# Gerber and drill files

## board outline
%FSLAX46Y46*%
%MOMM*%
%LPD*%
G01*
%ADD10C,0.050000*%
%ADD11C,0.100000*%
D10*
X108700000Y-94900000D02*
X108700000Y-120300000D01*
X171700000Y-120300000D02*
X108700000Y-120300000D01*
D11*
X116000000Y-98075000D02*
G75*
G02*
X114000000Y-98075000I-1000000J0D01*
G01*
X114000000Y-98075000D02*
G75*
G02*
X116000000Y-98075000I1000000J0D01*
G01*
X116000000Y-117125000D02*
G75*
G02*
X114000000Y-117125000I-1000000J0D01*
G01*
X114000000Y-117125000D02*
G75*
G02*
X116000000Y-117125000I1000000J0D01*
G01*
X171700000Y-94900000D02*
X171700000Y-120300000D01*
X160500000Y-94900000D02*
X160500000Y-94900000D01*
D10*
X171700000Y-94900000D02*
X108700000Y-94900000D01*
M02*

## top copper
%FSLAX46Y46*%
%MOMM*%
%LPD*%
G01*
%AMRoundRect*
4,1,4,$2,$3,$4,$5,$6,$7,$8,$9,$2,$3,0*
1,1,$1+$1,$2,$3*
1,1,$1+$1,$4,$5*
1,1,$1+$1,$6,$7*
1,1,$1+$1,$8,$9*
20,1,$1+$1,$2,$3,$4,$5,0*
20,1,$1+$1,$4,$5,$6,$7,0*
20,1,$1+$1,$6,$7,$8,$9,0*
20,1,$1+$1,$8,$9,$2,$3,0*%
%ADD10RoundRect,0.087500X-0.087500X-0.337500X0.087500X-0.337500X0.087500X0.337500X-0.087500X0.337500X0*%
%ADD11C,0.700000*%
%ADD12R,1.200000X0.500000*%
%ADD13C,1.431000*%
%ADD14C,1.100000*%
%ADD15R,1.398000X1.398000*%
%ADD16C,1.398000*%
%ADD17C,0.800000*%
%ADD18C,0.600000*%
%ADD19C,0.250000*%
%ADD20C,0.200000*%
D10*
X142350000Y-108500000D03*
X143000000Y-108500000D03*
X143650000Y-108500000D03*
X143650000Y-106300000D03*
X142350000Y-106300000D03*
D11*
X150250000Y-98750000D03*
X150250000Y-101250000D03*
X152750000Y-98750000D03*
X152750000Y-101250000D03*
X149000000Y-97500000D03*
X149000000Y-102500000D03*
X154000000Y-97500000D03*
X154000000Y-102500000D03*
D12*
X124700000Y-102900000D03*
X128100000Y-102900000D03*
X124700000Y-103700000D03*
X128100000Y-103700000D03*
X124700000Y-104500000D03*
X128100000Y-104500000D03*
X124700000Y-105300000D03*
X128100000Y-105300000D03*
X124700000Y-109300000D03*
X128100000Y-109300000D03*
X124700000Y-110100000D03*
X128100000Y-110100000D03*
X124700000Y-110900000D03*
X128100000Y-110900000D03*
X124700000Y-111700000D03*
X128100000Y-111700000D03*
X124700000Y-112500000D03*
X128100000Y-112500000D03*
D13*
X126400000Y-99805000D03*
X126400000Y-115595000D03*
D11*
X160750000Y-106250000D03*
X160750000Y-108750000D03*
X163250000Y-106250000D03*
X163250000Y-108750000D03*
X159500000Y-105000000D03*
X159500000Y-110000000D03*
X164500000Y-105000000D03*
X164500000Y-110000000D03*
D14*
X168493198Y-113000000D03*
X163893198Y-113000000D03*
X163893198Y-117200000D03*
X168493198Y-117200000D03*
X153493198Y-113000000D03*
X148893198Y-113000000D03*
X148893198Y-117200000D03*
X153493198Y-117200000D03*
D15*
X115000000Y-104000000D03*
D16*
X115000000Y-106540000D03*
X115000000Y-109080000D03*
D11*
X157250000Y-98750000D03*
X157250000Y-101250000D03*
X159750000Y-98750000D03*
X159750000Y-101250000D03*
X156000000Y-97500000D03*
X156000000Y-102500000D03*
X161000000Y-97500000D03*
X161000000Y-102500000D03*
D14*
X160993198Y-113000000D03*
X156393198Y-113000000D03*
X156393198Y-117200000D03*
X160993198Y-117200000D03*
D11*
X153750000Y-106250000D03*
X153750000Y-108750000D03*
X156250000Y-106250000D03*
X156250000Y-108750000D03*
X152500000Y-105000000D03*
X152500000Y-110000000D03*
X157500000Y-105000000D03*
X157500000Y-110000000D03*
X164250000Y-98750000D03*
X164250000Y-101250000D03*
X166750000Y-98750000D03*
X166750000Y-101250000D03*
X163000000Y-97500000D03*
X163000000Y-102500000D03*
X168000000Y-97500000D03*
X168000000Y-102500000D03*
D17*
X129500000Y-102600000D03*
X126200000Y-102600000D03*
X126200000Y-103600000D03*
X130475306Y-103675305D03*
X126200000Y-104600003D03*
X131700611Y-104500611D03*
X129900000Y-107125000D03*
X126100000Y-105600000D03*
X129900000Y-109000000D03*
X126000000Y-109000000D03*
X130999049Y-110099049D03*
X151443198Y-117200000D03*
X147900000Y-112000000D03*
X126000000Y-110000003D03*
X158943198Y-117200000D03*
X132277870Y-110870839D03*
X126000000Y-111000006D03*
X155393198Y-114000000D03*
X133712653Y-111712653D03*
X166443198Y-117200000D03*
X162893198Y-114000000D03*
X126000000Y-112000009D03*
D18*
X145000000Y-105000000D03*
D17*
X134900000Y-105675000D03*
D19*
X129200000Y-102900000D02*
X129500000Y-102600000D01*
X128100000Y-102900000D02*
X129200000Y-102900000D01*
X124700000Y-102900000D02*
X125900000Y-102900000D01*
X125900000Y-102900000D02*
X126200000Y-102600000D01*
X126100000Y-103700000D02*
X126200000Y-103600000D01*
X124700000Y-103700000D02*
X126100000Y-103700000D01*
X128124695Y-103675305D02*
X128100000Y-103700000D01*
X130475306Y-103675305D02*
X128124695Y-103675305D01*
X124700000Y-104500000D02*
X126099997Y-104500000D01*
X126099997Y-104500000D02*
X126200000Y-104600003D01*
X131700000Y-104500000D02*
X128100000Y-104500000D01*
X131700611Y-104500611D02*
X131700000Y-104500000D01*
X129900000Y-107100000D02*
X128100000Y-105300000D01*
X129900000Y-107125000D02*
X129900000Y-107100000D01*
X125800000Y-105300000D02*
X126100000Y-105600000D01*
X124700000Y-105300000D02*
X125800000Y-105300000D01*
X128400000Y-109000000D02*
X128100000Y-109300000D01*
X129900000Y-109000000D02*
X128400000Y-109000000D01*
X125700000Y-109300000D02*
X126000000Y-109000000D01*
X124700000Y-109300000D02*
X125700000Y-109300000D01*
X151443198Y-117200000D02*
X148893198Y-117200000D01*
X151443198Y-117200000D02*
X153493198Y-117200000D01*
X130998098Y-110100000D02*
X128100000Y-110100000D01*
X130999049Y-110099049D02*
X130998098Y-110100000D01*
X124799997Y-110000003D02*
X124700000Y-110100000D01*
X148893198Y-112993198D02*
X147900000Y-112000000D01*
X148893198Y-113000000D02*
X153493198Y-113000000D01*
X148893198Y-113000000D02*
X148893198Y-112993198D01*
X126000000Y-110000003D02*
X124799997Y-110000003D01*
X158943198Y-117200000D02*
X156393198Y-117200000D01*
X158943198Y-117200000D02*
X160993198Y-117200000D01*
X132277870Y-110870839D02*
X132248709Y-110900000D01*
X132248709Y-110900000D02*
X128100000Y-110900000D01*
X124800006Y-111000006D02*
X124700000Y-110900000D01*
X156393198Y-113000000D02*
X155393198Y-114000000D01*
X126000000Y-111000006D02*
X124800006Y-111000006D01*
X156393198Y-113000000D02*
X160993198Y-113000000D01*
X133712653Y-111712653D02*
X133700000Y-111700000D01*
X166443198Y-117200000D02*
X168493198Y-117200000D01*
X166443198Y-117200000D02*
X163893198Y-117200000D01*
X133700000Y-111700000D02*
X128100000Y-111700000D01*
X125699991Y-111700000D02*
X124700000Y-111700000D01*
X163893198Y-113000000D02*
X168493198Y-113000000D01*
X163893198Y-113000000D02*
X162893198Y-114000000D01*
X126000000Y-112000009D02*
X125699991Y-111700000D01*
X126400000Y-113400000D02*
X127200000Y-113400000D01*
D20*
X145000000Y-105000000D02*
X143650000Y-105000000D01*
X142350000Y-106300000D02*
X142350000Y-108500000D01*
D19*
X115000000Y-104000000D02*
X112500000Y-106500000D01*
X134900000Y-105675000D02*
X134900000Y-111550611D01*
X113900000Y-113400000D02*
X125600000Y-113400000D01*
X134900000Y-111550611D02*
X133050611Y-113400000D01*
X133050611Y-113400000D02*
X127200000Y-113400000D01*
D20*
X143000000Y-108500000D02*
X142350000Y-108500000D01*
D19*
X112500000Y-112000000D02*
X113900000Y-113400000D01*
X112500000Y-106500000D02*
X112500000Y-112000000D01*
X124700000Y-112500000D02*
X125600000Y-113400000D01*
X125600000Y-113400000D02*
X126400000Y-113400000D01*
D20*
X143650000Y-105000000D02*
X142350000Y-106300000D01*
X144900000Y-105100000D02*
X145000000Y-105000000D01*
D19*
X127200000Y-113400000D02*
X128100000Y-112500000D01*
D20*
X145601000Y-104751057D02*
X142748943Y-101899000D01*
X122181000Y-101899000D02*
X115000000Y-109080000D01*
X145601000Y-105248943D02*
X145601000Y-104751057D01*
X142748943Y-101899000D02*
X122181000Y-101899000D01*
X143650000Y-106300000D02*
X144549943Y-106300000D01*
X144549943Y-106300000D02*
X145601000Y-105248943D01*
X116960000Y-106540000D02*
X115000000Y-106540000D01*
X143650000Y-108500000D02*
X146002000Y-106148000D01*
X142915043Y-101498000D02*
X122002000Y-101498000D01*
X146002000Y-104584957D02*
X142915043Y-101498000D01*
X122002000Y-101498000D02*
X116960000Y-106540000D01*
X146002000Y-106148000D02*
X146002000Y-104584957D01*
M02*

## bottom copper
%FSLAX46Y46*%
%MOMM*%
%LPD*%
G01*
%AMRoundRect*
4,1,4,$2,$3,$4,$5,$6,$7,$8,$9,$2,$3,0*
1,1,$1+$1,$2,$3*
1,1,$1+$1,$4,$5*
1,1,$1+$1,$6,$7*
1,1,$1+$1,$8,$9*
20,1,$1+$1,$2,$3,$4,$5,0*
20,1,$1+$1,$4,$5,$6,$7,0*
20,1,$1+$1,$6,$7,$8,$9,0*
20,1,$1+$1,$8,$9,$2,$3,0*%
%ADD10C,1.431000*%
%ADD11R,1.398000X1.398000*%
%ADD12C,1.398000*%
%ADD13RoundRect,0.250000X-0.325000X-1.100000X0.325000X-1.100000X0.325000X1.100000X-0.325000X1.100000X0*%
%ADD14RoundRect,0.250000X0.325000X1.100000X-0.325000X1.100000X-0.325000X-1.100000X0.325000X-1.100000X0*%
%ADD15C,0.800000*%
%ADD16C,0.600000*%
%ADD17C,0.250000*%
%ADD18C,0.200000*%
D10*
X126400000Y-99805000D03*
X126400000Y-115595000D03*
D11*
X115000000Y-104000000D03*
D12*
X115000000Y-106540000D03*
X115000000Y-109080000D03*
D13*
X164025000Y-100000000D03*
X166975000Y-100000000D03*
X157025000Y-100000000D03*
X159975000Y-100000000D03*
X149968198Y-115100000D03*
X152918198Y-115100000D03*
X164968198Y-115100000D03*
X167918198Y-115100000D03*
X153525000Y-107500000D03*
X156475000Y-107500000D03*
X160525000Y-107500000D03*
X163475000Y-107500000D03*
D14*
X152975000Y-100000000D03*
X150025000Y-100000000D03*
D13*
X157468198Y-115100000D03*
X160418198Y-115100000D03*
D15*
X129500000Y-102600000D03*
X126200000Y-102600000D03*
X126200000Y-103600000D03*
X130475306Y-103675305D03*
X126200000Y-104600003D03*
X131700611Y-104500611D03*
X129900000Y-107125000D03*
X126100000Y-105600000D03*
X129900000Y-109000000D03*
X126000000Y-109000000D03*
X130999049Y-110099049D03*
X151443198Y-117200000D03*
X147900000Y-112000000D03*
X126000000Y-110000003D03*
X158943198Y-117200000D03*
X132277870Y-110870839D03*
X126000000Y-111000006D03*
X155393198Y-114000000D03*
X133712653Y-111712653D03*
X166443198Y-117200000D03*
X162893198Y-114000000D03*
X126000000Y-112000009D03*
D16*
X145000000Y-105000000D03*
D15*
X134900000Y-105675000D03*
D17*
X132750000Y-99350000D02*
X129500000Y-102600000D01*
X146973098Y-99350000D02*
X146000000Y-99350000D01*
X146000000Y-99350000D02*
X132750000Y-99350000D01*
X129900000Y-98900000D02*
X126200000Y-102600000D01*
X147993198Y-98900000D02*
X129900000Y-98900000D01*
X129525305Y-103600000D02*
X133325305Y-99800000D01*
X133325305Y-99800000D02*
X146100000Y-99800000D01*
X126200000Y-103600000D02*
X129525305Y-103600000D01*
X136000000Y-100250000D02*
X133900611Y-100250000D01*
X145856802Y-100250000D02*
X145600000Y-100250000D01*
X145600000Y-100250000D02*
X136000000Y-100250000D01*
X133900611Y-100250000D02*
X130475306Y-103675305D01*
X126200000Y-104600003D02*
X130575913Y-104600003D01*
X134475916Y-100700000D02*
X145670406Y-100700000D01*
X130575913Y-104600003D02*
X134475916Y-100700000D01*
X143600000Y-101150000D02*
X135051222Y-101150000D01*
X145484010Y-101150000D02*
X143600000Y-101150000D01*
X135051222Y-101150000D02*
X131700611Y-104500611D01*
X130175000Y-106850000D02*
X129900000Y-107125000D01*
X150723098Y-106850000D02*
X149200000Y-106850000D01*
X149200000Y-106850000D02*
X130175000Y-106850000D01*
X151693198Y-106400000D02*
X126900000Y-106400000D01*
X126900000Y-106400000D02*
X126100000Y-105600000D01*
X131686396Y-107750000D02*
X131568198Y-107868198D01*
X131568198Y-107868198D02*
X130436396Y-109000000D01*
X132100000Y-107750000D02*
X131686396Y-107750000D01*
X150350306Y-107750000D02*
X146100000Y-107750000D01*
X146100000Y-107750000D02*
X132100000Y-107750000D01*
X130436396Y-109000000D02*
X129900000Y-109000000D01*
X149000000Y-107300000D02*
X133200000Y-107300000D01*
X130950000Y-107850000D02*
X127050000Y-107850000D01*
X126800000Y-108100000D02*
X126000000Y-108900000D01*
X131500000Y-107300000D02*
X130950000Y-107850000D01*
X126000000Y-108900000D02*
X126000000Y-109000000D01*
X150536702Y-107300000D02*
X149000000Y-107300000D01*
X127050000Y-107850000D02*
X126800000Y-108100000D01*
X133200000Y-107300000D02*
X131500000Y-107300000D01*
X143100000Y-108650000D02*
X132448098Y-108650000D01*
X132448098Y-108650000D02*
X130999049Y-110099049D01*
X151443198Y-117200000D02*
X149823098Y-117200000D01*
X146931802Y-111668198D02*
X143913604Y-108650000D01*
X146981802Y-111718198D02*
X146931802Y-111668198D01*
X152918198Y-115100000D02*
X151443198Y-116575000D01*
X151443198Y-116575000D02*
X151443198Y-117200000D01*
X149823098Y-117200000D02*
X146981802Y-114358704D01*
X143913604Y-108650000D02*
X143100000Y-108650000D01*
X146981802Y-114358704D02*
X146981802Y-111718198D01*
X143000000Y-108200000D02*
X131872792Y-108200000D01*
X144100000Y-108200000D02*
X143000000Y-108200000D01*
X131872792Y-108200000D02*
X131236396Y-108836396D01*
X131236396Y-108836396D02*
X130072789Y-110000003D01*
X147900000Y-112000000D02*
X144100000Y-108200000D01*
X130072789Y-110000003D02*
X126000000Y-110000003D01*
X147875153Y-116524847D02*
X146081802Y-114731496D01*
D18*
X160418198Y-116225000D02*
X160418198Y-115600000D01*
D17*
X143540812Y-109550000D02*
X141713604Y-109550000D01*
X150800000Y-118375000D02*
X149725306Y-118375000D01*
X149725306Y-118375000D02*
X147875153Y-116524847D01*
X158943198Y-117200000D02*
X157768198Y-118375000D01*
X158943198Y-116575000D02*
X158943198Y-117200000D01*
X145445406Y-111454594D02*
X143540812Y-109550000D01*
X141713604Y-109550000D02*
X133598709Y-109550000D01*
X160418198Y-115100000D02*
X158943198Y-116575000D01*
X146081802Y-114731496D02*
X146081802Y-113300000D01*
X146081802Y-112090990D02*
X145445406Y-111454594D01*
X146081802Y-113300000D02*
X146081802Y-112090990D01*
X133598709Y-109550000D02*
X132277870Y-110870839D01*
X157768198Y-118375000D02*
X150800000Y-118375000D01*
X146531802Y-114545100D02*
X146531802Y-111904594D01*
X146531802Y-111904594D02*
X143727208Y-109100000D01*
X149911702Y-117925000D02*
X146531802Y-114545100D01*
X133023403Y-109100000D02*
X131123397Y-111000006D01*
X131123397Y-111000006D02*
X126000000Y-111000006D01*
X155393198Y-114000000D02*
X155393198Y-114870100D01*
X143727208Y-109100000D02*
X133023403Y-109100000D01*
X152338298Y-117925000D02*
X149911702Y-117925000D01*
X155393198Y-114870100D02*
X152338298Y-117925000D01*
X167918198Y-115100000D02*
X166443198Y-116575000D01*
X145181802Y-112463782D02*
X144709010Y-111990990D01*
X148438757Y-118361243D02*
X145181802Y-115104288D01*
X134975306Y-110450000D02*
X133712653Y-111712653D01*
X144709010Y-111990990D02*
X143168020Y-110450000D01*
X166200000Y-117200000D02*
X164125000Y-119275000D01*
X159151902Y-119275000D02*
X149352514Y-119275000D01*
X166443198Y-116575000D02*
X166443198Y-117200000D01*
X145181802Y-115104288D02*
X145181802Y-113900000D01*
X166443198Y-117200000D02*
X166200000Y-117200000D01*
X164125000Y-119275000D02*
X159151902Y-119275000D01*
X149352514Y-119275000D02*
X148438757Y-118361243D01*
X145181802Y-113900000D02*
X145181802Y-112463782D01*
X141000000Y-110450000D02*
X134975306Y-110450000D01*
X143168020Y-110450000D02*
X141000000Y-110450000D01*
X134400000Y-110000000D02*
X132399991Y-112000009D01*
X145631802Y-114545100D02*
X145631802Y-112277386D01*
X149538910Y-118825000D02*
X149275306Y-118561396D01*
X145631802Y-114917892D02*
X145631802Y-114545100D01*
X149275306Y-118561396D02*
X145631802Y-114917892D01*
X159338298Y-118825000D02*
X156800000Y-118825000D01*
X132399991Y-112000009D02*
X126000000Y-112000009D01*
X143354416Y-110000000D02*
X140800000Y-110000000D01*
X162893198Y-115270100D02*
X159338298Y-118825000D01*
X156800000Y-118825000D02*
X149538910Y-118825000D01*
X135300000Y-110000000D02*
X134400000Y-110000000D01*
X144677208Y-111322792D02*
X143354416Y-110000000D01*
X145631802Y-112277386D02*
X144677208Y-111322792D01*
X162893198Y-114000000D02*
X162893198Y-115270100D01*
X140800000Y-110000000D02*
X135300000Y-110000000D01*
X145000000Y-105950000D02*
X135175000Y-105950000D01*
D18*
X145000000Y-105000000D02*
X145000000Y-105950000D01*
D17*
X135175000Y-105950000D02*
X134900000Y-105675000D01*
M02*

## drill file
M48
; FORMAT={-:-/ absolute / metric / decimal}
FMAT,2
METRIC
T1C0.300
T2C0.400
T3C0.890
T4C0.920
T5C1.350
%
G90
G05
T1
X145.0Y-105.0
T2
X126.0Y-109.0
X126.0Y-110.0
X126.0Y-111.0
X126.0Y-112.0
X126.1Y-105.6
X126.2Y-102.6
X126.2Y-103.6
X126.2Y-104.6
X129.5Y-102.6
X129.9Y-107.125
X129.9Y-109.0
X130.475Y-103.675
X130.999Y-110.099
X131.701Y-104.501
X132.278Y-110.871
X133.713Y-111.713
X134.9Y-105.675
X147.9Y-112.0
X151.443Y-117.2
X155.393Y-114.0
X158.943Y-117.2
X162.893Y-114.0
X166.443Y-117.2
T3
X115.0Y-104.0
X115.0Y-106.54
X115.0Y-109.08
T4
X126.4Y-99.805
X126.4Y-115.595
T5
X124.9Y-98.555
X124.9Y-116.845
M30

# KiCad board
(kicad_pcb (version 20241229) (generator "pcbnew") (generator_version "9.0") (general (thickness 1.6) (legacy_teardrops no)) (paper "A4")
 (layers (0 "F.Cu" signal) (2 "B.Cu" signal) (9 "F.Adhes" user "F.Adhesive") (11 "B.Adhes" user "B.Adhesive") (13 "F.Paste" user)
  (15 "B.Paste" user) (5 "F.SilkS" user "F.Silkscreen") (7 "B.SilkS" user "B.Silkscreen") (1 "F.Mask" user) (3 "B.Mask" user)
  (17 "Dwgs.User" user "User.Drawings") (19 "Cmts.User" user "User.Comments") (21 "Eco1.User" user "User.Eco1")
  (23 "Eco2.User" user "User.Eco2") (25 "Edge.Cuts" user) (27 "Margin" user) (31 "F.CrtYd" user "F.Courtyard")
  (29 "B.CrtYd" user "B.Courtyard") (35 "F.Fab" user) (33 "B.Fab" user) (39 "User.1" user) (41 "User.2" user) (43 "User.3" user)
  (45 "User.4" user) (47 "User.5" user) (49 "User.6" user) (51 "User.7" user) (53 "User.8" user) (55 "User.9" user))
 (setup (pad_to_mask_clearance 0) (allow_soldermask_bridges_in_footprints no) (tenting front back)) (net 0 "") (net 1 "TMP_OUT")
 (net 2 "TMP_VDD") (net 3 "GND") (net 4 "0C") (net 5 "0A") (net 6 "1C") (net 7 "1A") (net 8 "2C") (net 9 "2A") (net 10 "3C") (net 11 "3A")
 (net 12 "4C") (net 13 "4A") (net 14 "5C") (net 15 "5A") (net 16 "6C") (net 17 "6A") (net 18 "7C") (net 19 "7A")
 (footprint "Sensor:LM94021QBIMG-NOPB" (layer "F.Cu") (at 143 107.4)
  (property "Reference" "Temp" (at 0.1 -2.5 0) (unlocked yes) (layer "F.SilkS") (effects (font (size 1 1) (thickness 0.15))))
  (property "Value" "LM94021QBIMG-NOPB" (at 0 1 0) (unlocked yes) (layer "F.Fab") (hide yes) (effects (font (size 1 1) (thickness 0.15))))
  (pad "1" smd roundrect (at -0.65 1.1) (size 0.35 0.85) (layers "F.Cu" "F.Mask" "F.Paste") (roundrect_rratio 0.25))
  (pad "2" smd roundrect (at 0 1.1) (size 0.35 0.85) (layers "F.Cu" "F.Mask" "F.Paste") (roundrect_rratio 0.25))
  (pad "3" smd roundrect (at 0.65 1.1) (size 0.35 0.85) (layers "F.Cu" "F.Mask" "F.Paste") (roundrect_rratio 0.25) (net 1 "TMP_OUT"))
  (pad "4" smd roundrect (at 0.65 -1.1) (size 0.35 0.85) (layers "F.Cu" "F.Mask" "F.Paste") (roundrect_rratio 0.25) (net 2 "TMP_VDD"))
  (pad "5" smd roundrect (at -0.65 -1.1) (size 0.35 0.85) (layers "F.Cu" "F.Mask" "F.Paste") (roundrect_rratio 0.25) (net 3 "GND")))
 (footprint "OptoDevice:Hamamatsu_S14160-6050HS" (layer "F.Cu") (at 151.5 100)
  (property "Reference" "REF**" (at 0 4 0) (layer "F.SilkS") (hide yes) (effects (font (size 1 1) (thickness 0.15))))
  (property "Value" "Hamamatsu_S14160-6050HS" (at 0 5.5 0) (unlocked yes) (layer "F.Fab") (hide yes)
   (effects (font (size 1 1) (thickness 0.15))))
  (pad "A" smd circle (at -1.25 -1.25) (size 0.7 0.7) (layers "F.Cu" "F.Mask" "F.Paste"))
  (pad "A" smd circle (at -1.25 1.25) (size 0.7 0.7) (layers "F.Cu" "F.Mask" "F.Paste"))
  (pad "A" smd circle (at 1.25 -1.25) (size 0.7 0.7) (layers "F.Cu" "F.Mask" "F.Paste"))
  (pad "A" smd circle (at 1.25 1.25) (size 0.7 0.7) (layers "F.Cu" "F.Mask" "F.Paste"))
  (pad "K" smd circle (at -2.5 -2.5) (size 0.7 0.7) (layers "F.Cu" "F.Mask" "F.Paste"))
  (pad "K" smd circle (at -2.5 2.5) (size 0.7 0.7) (layers "F.Cu" "F.Mask" "F.Paste"))
  (pad "K" smd circle (at 2.5 -2.5) (size 0.7 0.7) (layers "F.Cu" "F.Mask" "F.Paste"))
  (pad "K" smd circle (at 2.5 2.5) (size 0.7 0.7) (layers "F.Cu" "F.Mask" "F.Paste")))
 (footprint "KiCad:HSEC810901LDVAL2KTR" (layer "F.Cu") (at 126.4 107.7 -90)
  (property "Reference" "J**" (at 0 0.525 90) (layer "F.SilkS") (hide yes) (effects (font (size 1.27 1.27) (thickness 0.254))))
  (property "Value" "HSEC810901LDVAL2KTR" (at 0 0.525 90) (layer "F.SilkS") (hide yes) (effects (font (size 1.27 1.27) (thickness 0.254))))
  (pad "" np_thru_hole circle (at -9.145 1.5 270) (size 1.35 1.35) (drill 1.35) (layers "*.Cu" "*.Mask"))
  (pad "" np_thru_hole circle (at 9.145 1.5 270) (size 1.35 1.35) (drill 1.35) (layers "*.Cu" "*.Mask"))
  (pad "1" smd rect (at -4.8 1.7 270) (size 0.5 1.2) (layers "F.Cu" "F.Mask" "F.Paste") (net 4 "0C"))
  (pad "2" smd rect (at -4.8 -1.7 270) (size 0.5 1.2) (layers "F.Cu" "F.Mask" "F.Paste") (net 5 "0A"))
  (pad "3" smd rect (at -4 1.7 270) (size 0.5 1.2) (layers "F.Cu" "F.Mask" "F.Paste") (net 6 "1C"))
  (pad "4" smd rect (at -4 -1.7 270) (size 0.5 1.2) (layers "F.Cu" "F.Mask" "F.Paste") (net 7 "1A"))
  (pad "5" smd rect (at -3.2 1.7 270) (size 0.5 1.2) (layers "F.Cu" "F.Mask" "F.Paste") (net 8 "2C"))
  (pad "6" smd rect (at -3.2 -1.7 270) (size 0.5 1.2) (layers "F.Cu" "F.Mask" "F.Paste") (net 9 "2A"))
  (pad "7" smd rect (at -2.4 1.7 270) (size 0.5 1.2) (layers "F.Cu" "F.Mask" "F.Paste") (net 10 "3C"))
  (pad "8" smd rect (at -2.4 -1.7 270) (size 0.5 1.2) (layers "F.Cu" "F.Mask" "F.Paste") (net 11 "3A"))
  (pad "9" smd rect (at 1.6 1.7 270) (size 0.5 1.2) (layers "F.Cu" "F.Mask" "F.Paste") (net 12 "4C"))
  (pad "10" smd rect (at 1.6 -1.7 270) (size 0.5 1.2) (layers "F.Cu" "F.Mask" "F.Paste") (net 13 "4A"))
  (pad "11" smd rect (at 2.4 1.7 270) (size 0.5 1.2) (layers "F.Cu" "F.Mask" "F.Paste") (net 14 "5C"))
  (pad "12" smd rect (at 2.4 -1.7 270) (size 0.5 1.2) (layers "F.Cu" "F.Mask" "F.Paste") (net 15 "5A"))
  (pad "13" smd rect (at 3.2 1.7 270) (size 0.5 1.2) (layers "F.Cu" "F.Mask" "F.Paste") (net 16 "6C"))
  (pad "14" smd rect (at 3.2 -1.7 270) (size 0.5 1.2) (layers "F.Cu" "F.Mask" "F.Paste") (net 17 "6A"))
  (pad "15" smd rect (at 4 1.7 270) (size 0.5 1.2) (layers "F.Cu" "F.Mask" "F.Paste") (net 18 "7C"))
  (pad "16" smd rect (at 4 -1.7 270) (size 0.5 1.2) (layers "F.Cu" "F.Mask" "F.Paste") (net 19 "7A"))
  (pad "17" smd rect (at 4.8 1.7 270) (size 0.5 1.2) (layers "F.Cu" "F.Mask" "F.Paste") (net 3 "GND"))
  (pad "18" smd rect (at 4.8 -1.7 270) (size 0.5 1.2) (layers "F.Cu" "F.Mask" "F.Paste") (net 3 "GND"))
  (pad "MH1" thru_hole circle (at -7.895 0 270) (size 1.431 1.431) (drill 0.92) (layers "*.Cu" "*.Mask") (remove_unused_layers no))
  (pad "MH2" thru_hole circle (at 7.895 0 270) (size 1.431 1.431) (drill 0.92) (layers "*.Cu" "*.Mask") (remove_unused_layers no)))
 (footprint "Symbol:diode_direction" (layer "F.Cu") (at 150.243198 107.6 90)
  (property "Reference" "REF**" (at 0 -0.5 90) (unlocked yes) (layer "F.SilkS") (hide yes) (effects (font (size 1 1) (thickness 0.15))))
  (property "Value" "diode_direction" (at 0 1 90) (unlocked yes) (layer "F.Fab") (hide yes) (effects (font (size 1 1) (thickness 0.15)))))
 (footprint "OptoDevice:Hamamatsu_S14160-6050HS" (layer "F.Cu") (at 162 107.5)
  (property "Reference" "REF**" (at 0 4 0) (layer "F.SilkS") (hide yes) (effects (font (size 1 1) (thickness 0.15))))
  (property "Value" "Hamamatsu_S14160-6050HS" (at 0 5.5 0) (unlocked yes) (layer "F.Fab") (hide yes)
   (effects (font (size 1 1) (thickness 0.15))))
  (pad "A" smd circle (at -1.25 -1.25) (size 0.7 0.7) (layers "F.Cu" "F.Mask" "F.Paste"))
  (pad "A" smd circle (at -1.25 1.25) (size 0.7 0.7) (layers "F.Cu" "F.Mask" "F.Paste"))
  (pad "A" smd circle (at 1.25 -1.25) (size 0.7 0.7) (layers "F.Cu" "F.Mask" "F.Paste"))
  (pad "A" smd circle (at 1.25 1.25) (size 0.7 0.7) (layers "F.Cu" "F.Mask" "F.Paste"))
  (pad "K" smd circle (at -2.5 -2.5) (size 0.7 0.7) (layers "F.Cu" "F.Mask" "F.Paste"))
  (pad "K" smd circle (at -2.5 2.5) (size 0.7 0.7) (layers "F.Cu" "F.Mask" "F.Paste"))
  (pad "K" smd circle (at 2.5 -2.5) (size 0.7 0.7) (layers "F.Cu" "F.Mask" "F.Paste"))
  (pad "K" smd circle (at 2.5 2.5) (size 0.7 0.7) (layers "F.Cu" "F.Mask" "F.Paste")))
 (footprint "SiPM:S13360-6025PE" (layer "F.Cu") (at 166.443198 115.1)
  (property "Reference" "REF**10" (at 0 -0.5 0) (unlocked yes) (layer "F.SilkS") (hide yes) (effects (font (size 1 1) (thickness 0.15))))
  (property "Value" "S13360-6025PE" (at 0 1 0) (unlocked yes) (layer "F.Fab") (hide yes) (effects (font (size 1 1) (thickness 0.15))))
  (pad "1" smd circle (at 2.05 -2.1) (size 1.1 1.1) (layers "F.Cu" "F.Mask" "F.Paste") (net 18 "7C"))
  (pad "2" smd circle (at -2.55 -2.1) (size 1.1 1.1) (layers "F.Cu" "F.Mask" "F.Paste") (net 18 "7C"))
  (pad "3" smd circle (at -2.55 2.1) (size 1.1 1.1) (layers "F.Cu" "F.Mask" "F.Paste") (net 19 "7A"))
  (pad "4" smd circle (at 2.05 2.1) (size 1.1 1.1) (layers "F.Cu" "F.Mask" "F.Paste") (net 19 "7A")))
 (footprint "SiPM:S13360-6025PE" (layer "F.Cu") (at 151.443198 115.1)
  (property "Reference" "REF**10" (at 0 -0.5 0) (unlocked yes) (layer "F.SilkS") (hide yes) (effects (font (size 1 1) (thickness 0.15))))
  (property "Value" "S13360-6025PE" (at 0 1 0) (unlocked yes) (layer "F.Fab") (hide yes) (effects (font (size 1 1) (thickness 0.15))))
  (pad "1" smd circle (at 2.05 -2.1) (size 1.1 1.1) (layers "F.Cu" "F.Mask" "F.Paste") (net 14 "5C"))
  (pad "2" smd circle (at -2.55 -2.1) (size 1.1 1.1) (layers "F.Cu" "F.Mask" "F.Paste") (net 14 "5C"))
  (pad "3" smd circle (at -2.55 2.1) (size 1.1 1.1) (layers "F.Cu" "F.Mask" "F.Paste") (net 15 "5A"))
  (pad "4" smd circle (at 2.05 2.1) (size 1.1 1.1) (layers "F.Cu" "F.Mask" "F.Paste") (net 15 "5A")))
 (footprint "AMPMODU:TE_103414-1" (layer "F.Cu") (at 115 106.54 -90)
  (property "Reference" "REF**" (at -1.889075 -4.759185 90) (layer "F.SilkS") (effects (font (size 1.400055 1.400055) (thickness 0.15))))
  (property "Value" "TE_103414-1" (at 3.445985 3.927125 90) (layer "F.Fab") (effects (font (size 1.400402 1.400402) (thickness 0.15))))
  (pad "1" thru_hole rect (at -2.54 0 270) (size 1.398 1.398) (drill 0.89) (layers "*.Cu" "*.Mask") (remove_unused_layers no) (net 3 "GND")
   (solder_mask_margin 0.102))
  (pad "2" thru_hole circle (at 0 0 270) (size 1.398 1.398) (drill 0.89) (layers "*.Cu" "*.Mask") (remove_unused_layers no)
   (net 1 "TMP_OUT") (solder_mask_margin 0.102))
  (pad "3" thru_hole circle (at 2.54 0 270) (size 1.398 1.398) (drill 0.89) (layers "*.Cu" "*.Mask") (remove_unused_layers no)
   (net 2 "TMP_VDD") (solder_mask_margin 0.102)))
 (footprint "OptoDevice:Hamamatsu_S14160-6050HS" (layer "F.Cu") (at 158.5 100)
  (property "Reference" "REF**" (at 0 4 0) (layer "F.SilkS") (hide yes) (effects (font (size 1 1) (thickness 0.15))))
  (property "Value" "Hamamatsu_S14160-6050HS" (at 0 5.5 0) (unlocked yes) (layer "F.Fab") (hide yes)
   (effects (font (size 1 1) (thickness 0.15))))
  (pad "A" smd circle (at -1.25 -1.25) (size 0.7 0.7) (layers "F.Cu" "F.Mask" "F.Paste"))
  (pad "A" smd circle (at -1.25 1.25) (size 0.7 0.7) (layers "F.Cu" "F.Mask" "F.Paste"))
  (pad "A" smd circle (at 1.25 -1.25) (size 0.7 0.7) (layers "F.Cu" "F.Mask" "F.Paste"))
  (pad "A" smd circle (at 1.25 1.25) (size 0.7 0.7) (layers "F.Cu" "F.Mask" "F.Paste"))
  (pad "K" smd circle (at -2.5 -2.5) (size 0.7 0.7) (layers "F.Cu" "F.Mask" "F.Paste"))
  (pad "K" smd circle (at -2.5 2.5) (size 0.7 0.7) (layers "F.Cu" "F.Mask" "F.Paste"))
  (pad "K" smd circle (at 2.5 -2.5) (size 0.7 0.7) (layers "F.Cu" "F.Mask" "F.Paste"))
  (pad "K" smd circle (at 2.5 2.5) (size 0.7 0.7) (layers "F.Cu" "F.Mask" "F.Paste")))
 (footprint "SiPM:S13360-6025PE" (layer "F.Cu") (at 158.943198 115.1)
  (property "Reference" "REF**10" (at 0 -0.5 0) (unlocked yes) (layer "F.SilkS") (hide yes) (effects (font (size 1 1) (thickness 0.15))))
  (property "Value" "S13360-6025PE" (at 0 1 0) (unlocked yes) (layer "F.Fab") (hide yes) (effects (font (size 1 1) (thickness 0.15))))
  (pad "1" smd circle (at 2.05 -2.1) (size 1.1 1.1) (layers "F.Cu" "F.Mask" "F.Paste") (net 16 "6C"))
  (pad "2" smd circle (at -2.55 -2.1) (size 1.1 1.1) (layers "F.Cu" "F.Mask" "F.Paste") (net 16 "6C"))
  (pad "3" smd circle (at -2.55 2.1) (size 1.1 1.1) (layers "F.Cu" "F.Mask" "F.Paste") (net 17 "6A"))
  (pad "4" smd circle (at 2.05 2.1) (size 1.1 1.1) (layers "F.Cu" "F.Mask" "F.Paste") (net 17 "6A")))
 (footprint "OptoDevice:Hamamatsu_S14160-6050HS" (layer "F.Cu") (at 155 107.5)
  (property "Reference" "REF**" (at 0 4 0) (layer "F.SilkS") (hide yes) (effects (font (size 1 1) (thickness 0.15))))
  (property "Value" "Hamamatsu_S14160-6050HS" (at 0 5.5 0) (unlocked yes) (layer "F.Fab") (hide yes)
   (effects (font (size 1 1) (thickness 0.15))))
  (pad "A" smd circle (at -1.25 -1.25) (size 0.7 0.7) (layers "F.Cu" "F.Mask" "F.Paste"))
  (pad "A" smd circle (at -1.25 1.25) (size 0.7 0.7) (layers "F.Cu" "F.Mask" "F.Paste"))
  (pad "A" smd circle (at 1.25 -1.25) (size 0.7 0.7) (layers "F.Cu" "F.Mask" "F.Paste"))
  (pad "A" smd circle (at 1.25 1.25) (size 0.7 0.7) (layers "F.Cu" "F.Mask" "F.Paste"))
  (pad "K" smd circle (at -2.5 -2.5) (size 0.7 0.7) (layers "F.Cu" "F.Mask" "F.Paste"))
  (pad "K" smd circle (at -2.5 2.5) (size 0.7 0.7) (layers "F.Cu" "F.Mask" "F.Paste"))
  (pad "K" smd circle (at 2.5 -2.5) (size 0.7 0.7) (layers "F.Cu" "F.Mask" "F.Paste"))
  (pad "K" smd circle (at 2.5 2.5) (size 0.7 0.7) (layers "F.Cu" "F.Mask" "F.Paste")))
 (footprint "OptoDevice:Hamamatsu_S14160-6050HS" (layer "F.Cu") (at 165.5 100)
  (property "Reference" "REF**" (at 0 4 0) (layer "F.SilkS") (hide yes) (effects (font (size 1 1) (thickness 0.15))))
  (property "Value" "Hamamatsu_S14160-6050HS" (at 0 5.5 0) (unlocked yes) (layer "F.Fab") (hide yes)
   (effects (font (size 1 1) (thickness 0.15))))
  (pad "A" smd circle (at -1.25 -1.25) (size 0.7 0.7) (layers "F.Cu" "F.Mask" "F.Paste"))
  (pad "A" smd circle (at -1.25 1.25) (size 0.7 0.7) (layers "F.Cu" "F.Mask" "F.Paste"))
  (pad "A" smd circle (at 1.25 -1.25) (size 0.7 0.7) (layers "F.Cu" "F.Mask" "F.Paste"))
  (pad "A" smd circle (at 1.25 1.25) (size 0.7 0.7) (layers "F.Cu" "F.Mask" "F.Paste"))
  (pad "K" smd circle (at -2.5 -2.5) (size 0.7 0.7) (layers "F.Cu" "F.Mask" "F.Paste"))
  (pad "K" smd circle (at -2.5 2.5) (size 0.7 0.7) (layers "F.Cu" "F.Mask" "F.Paste"))
  (pad "K" smd circle (at 2.5 -2.5) (size 0.7 0.7) (layers "F.Cu" "F.Mask" "F.Paste"))
  (pad "K" smd circle (at 2.5 2.5) (size 0.7 0.7) (layers "F.Cu" "F.Mask" "F.Paste")))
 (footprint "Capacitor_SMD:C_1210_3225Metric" (layer "B.Cu") (at 165.5 100)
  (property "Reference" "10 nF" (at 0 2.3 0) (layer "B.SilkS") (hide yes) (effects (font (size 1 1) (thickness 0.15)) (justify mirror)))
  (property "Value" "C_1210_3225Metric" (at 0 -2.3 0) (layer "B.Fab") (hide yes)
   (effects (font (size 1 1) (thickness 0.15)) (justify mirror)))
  (pad "1" smd roundrect (at -1.475 0) (size 1.15 2.7) (layers "B.Cu" "B.Mask" "B.Paste") (roundrect_rratio 0.2173913043) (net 3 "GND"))
  (pad "2" smd roundrect (at 1.475 0) (size 1.15 2.7) (layers "B.Cu" "B.Mask" "B.Paste") (roundrect_rratio 0.2173913043) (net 9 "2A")))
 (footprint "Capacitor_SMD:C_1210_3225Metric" (layer "B.Cu") (at 158.5 100)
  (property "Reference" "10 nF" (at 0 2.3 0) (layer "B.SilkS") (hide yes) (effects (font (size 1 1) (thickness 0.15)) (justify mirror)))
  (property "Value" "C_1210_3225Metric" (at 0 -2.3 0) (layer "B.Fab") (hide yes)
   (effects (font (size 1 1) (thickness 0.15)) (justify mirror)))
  (pad "1" smd roundrect (at -1.475 0) (size 1.15 2.7) (layers "B.Cu" "B.Mask" "B.Paste") (roundrect_rratio 0.2173913043) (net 3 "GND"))
  (pad "2" smd roundrect (at 1.475 0) (size 1.15 2.7) (layers "B.Cu" "B.Mask" "B.Paste") (roundrect_rratio 0.2173913043) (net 7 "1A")))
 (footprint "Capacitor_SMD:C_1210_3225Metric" (layer "B.Cu") (at 151.443198 115.1)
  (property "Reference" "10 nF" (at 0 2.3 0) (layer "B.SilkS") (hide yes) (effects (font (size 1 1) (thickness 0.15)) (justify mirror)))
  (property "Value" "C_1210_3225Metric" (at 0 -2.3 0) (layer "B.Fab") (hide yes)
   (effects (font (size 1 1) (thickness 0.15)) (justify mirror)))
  (pad "1" smd roundrect (at -1.475 0) (size 1.15 2.7) (layers "B.Cu" "B.Mask" "B.Paste") (roundrect_rratio 0.2173913043) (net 3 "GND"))
  (pad "2" smd roundrect (at 1.475 0) (size 1.15 2.7) (layers "B.Cu" "B.Mask" "B.Paste") (roundrect_rratio 0.2173913043) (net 15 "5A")))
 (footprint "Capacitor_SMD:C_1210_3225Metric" (layer "B.Cu") (at 166.443198 115.1)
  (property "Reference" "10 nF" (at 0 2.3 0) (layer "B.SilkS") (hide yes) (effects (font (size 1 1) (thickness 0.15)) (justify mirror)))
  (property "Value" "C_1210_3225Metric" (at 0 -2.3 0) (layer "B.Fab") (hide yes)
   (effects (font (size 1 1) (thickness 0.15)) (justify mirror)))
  (pad "1" smd roundrect (at -1.475 0) (size 1.15 2.7) (layers "B.Cu" "B.Mask" "B.Paste") (roundrect_rratio 0.2173913043) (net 3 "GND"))
  (pad "2" smd roundrect (at 1.475 0) (size 1.15 2.7) (layers "B.Cu" "B.Mask" "B.Paste") (roundrect_rratio 0.2173913043) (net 19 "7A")))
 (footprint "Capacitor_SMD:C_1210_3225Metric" (layer "B.Cu") (at 155 107.5)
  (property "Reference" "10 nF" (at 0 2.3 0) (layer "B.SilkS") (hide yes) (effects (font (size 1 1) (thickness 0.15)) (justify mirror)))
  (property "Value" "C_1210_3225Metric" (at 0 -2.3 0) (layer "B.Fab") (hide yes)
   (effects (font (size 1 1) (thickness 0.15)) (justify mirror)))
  (pad "1" smd roundrect (at -1.475 0) (size 1.15 2.7) (layers "B.Cu" "B.Mask" "B.Paste") (roundrect_rratio 0.2173913043) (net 3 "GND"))
  (pad "2" smd roundrect (at 1.475 0) (size 1.15 2.7) (layers "B.Cu" "B.Mask" "B.Paste") (roundrect_rratio 0.2173913043) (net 11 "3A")))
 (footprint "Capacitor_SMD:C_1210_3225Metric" (layer "B.Cu") (at 162 107.5)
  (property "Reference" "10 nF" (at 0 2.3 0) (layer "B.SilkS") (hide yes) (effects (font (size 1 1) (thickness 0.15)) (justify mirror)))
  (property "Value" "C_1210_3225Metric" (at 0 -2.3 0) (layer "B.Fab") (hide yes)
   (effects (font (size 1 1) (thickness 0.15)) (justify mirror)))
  (pad "1" smd roundrect (at -1.475 0) (size 1.15 2.7) (layers "B.Cu" "B.Mask" "B.Paste") (roundrect_rratio 0.2173913043) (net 3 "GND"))
  (pad "2" smd roundrect (at 1.475 0) (size 1.15 2.7) (layers "B.Cu" "B.Mask" "B.Paste") (roundrect_rratio 0.2173913043) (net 13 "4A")))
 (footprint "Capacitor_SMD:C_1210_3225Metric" (layer "B.Cu") (at 151.5 100 180)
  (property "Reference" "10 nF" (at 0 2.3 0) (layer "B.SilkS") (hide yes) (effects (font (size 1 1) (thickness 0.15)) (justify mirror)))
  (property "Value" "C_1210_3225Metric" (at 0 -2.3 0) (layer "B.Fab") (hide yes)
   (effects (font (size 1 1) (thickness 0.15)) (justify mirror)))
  (pad "1" smd roundrect (at -1.475 0 180) (size 1.15 2.7) (layers "B.Cu" "B.Mask" "B.Paste") (roundrect_rratio 0.2173913043) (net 5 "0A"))
  (pad "2" smd roundrect (at 1.475 0 180) (size 1.15 2.7) (layers "B.Cu" "B.Mask" "B.Paste") (roundrect_rratio 0.2173913043) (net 3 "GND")))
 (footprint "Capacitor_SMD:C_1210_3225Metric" (layer "B.Cu") (at 158.943198 115.1)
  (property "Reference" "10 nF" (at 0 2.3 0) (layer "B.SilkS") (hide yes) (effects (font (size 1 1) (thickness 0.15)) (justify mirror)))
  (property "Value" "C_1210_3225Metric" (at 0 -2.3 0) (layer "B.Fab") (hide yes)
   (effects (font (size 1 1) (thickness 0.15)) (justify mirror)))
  (pad "1" smd roundrect (at -1.475 0) (size 1.15 2.7) (layers "B.Cu" "B.Mask" "B.Paste") (roundrect_rratio 0.2173913043) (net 3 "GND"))
  (pad "2" smd roundrect (at 1.475 0) (size 1.15 2.7) (layers "B.Cu" "B.Mask" "B.Paste") (roundrect_rratio 0.2173913043) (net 17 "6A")))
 (gr_line (start 108.7 94.9) (end 108.7 120.3) (stroke (width 0.05) (type default)) (layer "Edge.Cuts"))
 (gr_line (start 171.7 120.3) (end 108.7 120.3) (stroke (width 0.05) (type solid)) (layer "Edge.Cuts"))
 (gr_circle (center 115 98.075) (end 116 98.075) (stroke (width 0.1) (type solid)) (fill no) (layer "Edge.Cuts"))
 (gr_circle (center 115 117.125) (end 116 117.125) (stroke (width 0.1) (type solid)) (fill no) (layer "Edge.Cuts"))
 (gr_line (start 171.7 94.9) (end 171.7 120.3) (stroke (width 0.1) (type default)) (layer "Edge.Cuts"))
 (gr_line (start 160.5 94.9) (end 160.5 94.9) (stroke (width 0.1) (type default)) (layer "Edge.Cuts"))
 (gr_line (start 171.7 94.9) (end 108.7 94.9) (stroke (width 0.05) (type solid)) (layer "Edge.Cuts"))
 (segment (start 129.2 102.9) (end 129.5 102.6) (width 0.25) (layer "F.Cu") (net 5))
 (segment (start 128.1 102.9) (end 129.2 102.9) (width 0.25) (layer "F.Cu") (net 5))
 (via (at 129.5 102.6) (size 0.8) (drill 0.4) (layers "F.Cu" "B.Cu") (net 5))
 (segment (start 132.75 99.35) (end 129.5 102.6) (width 0.25) (layer "B.Cu") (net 5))
 (segment (start 146.973098 99.35) (end 146 99.35) (width 0.25) (layer "B.Cu") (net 5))
 (segment (start 146 99.35) (end 132.75 99.35) (width 0.25) (layer "B.Cu") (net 5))
 (segment (start 124.7 102.9) (end 125.9 102.9) (width 0.25) (layer "F.Cu") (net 4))
 (segment (start 125.9 102.9) (end 126.2 102.6) (width 0.25) (layer "F.Cu") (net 4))
 (via (at 126.2 102.6) (size 0.8) (drill 0.4) (layers "F.Cu" "B.Cu") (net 4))
 (segment (start 129.9 98.9) (end 126.2 102.6) (width 0.25) (layer "B.Cu") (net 4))
 (segment (start 147.993198 98.9) (end 129.9 98.9) (width 0.25) (layer "B.Cu") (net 4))
 (segment (start 126.1 103.7) (end 126.2 103.6) (width 0.25) (layer "F.Cu") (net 6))
 (segment (start 124.7 103.7) (end 126.1 103.7) (width 0.25) (layer "F.Cu") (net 6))
 (via (at 126.2 103.6) (size 0.8) (drill 0.4) (layers "F.Cu" "B.Cu") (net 6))
 (segment (start 129.525305 103.6) (end 133.325305 99.8) (width 0.25) (layer "B.Cu") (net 6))
 (segment (start 133.325305 99.8) (end 146.1 99.8) (width 0.25) (layer "B.Cu") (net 6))
 (segment (start 126.2 103.6) (end 129.525305 103.6) (width 0.25) (layer "B.Cu") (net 6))
 (segment (start 128.124695 103.675305) (end 128.1 103.7) (width 0.25) (layer "F.Cu") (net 7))
 (segment (start 130.475306 103.675305) (end 128.124695 103.675305) (width 0.25) (layer "F.Cu") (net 7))
 (via (at 130.475306 103.675305) (size 0.8) (drill 0.4) (layers "F.Cu" "B.Cu") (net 7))
 (segment (start 136 100.25) (end 133.900611 100.25) (width 0.25) (layer "B.Cu") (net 7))
 (segment (start 145.856802 100.25) (end 145.6 100.25) (width 0.25) (layer "B.Cu") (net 7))
 (segment (start 145.6 100.25) (end 136 100.25) (width 0.25) (layer "B.Cu") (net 7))
 (segment (start 133.900611 100.25) (end 130.475306 103.675305) (width 0.25) (layer "B.Cu") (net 7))
 (segment (start 124.7 104.5) (end 126.099997 104.5) (width 0.25) (layer "F.Cu") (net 8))
 (segment (start 126.099997 104.5) (end 126.2 104.600003) (width 0.25) (layer "F.Cu") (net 8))
 (via (at 126.2 104.600003) (size 0.8) (drill 0.4) (layers "F.Cu" "B.Cu") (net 8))
 (segment (start 126.2 104.600003) (end 130.575913 104.600003) (width 0.25) (layer "B.Cu") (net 8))
 (segment (start 134.475916 100.7) (end 145.670406 100.7) (width 0.25) (layer "B.Cu") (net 8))
 (segment (start 130.575913 104.600003) (end 134.475916 100.7) (width 0.25) (layer "B.Cu") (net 8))
 (segment (start 131.7 104.5) (end 128.1 104.5) (width 0.25) (layer "F.Cu") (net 9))
 (segment (start 131.700611 104.500611) (end 131.7 104.5) (width 0.25) (layer "F.Cu") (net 9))
 (via (at 131.700611 104.500611) (size 0.8) (drill 0.4) (layers "F.Cu" "B.Cu") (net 9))
 (segment (start 143.6 101.15) (end 135.051222 101.15) (width 0.25) (layer "B.Cu") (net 9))
 (segment (start 145.48401 101.15) (end 143.6 101.15) (width 0.25) (layer "B.Cu") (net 9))
 (segment (start 135.051222 101.15) (end 131.700611 104.500611) (width 0.25) (layer "B.Cu") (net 9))
 (segment (start 129.9 107.1) (end 128.1 105.3) (width 0.25) (layer "F.Cu") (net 11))
 (segment (start 129.9 107.125) (end 129.9 107.1) (width 0.25) (layer "F.Cu") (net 11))
 (via (at 129.9 107.125) (size 0.8) (drill 0.4) (layers "F.Cu" "B.Cu") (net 11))
 (segment (start 130.175 106.85) (end 129.9 107.125) (width 0.25) (layer "B.Cu") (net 11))
 (segment (start 150.723098 106.85) (end 149.2 106.85) (width 0.25) (layer "B.Cu") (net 11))
 (segment (start 149.2 106.85) (end 130.175 106.85) (width 0.25) (layer "B.Cu") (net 11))
 (segment (start 125.8 105.3) (end 126.1 105.6) (width 0.25) (layer "F.Cu") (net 10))
 (segment (start 124.7 105.3) (end 125.8 105.3) (width 0.25) (layer "F.Cu") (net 10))
 (via (at 126.1 105.6) (size 0.8) (drill 0.4) (layers "F.Cu" "B.Cu") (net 10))
 (segment (start 151.693198 106.4) (end 126.9 106.4) (width 0.25) (layer "B.Cu") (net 10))
 (segment (start 126.9 106.4) (end 126.1 105.6) (width 0.25) (layer "B.Cu") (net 10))
 (segment (start 128.4 109) (end 128.1 109.3) (width 0.25) (layer "F.Cu") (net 13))
 (segment (start 129.9 109) (end 128.4 109) (width 0.25) (layer "F.Cu") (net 13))
 (via (at 129.9 109) (size 0.8) (drill 0.4) (layers "F.Cu" "B.Cu") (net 13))
 (segment (start 131.686396 107.75) (end 131.568198 107.868198) (width 0.25) (layer "B.Cu") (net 13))
 (segment (start 131.568198 107.868198) (end 130.436396 109) (width 0.25) (layer "B.Cu") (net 13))
 (segment (start 132.1 107.75) (end 131.686396 107.75) (width 0.25) (layer "B.Cu") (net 13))
 (segment (start 150.350306 107.75) (end 146.1 107.75) (width 0.25) (layer "B.Cu") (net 13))
 (segment (start 146.1 107.75) (end 132.1 107.75) (width 0.25) (layer "B.Cu") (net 13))
 (segment (start 130.436396 109) (end 129.9 109) (width 0.25) (layer "B.Cu") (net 13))
 (segment (start 125.7 109.3) (end 126 109) (width 0.25) (layer "F.Cu") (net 12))
 (segment (start 124.7 109.3) (end 125.7 109.3) (width 0.25) (layer "F.Cu") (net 12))
 (via (at 126 109) (size 0.8) (drill 0.4) (layers "F.Cu" "B.Cu") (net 12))
 (segment (start 149 107.3) (end 133.2 107.3) (width 0.25) (layer "B.Cu") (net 12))
 (segment (start 130.95 107.85) (end 127.05 107.85) (width 0.25) (layer "B.Cu") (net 12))
 (segment (start 126.8 108.1) (end 126 108.9) (width 0.25) (layer "B.Cu") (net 12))
 (segment (start 131.5 107.3) (end 130.95 107.85) (width 0.25) (layer "B.Cu") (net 12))
 (segment (start 126 108.9) (end 126 109) (width 0.25) (layer "B.Cu") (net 12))
 (segment (start 150.536702 107.3) (end 149 107.3) (width 0.25) (layer "B.Cu") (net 12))
 (segment (start 127.05 107.85) (end 126.8 108.1) (width 0.25) (layer "B.Cu") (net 12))
 (segment (start 133.2 107.3) (end 131.5 107.3) (width 0.25) (layer "B.Cu") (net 12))
 (segment (start 151.443198 117.2) (end 148.893198 117.2) (width 0.25) (layer "F.Cu") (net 15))
 (segment (start 151.443198 117.2) (end 153.493198 117.2) (width 0.25) (layer "F.Cu") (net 15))
 (segment (start 130.998098 110.1) (end 128.1 110.1) (width 0.25) (layer "F.Cu") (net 15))
 (segment (start 130.999049 110.099049) (end 130.998098 110.1) (width 0.25) (layer "F.Cu") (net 15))
 (via (at 130.999049 110.099049) (size 0.8) (drill 0.4) (layers "F.Cu" "B.Cu") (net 15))
 (via (at 151.443198 117.2) (size 0.8) (drill 0.4) (layers "F.Cu" "B.Cu") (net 15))
 (segment (start 143.1 108.65) (end 132.448098 108.65) (width 0.25) (layer "B.Cu") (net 15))
 (segment (start 132.448098 108.65) (end 130.999049 110.099049) (width 0.25) (layer "B.Cu") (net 15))
 (segment (start 151.443198 117.2) (end 149.823098 117.2) (width 0.25) (layer "B.Cu") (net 15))
 (segment (start 146.931802 111.668198) (end 143.913604 108.65) (width 0.25) (layer "B.Cu") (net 15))
 (segment (start 146.981802 111.718198) (end 146.931802 111.668198) (width 0.25) (layer "B.Cu") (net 15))
 (segment (start 152.918198 115.1) (end 151.443198 116.575) (width 0.25) (layer "B.Cu") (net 15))
 (segment (start 151.443198 116.575) (end 151.443198 117.2) (width 0.25) (layer "B.Cu") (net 15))
 (segment (start 149.823098 117.2) (end 146.981802 114.358704) (width 0.25) (layer "B.Cu") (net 15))
 (segment (start 143.913604 108.65) (end 143.1 108.65) (width 0.25) (layer "B.Cu") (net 15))
 (segment (start 146.981802 114.358704) (end 146.981802 111.718198) (width 0.25) (layer "B.Cu") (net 15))
 (segment (start 124.799997 110.000003) (end 124.7 110.1) (width 0.25) (layer "F.Cu") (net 14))
 (segment (start 148.893198 112.993198) (end 147.9 112) (width 0.25) (layer "F.Cu") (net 14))
 (segment (start 148.893198 113) (end 153.493198 113) (width 0.25) (layer "F.Cu") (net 14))
 (segment (start 148.893198 113) (end 148.893198 112.993198) (width 0.25) (layer "F.Cu") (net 14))
 (segment (start 126 110.000003) (end 124.799997 110.000003) (width 0.25) (layer "F.Cu") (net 14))
 (via (at 147.9 112) (size 0.8) (drill 0.4) (layers "F.Cu" "B.Cu") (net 14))
 (via (at 126 110.000003) (size 0.8) (drill 0.4) (layers "F.Cu" "B.Cu") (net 14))
 (segment (start 143 108.2) (end 131.872792 108.2) (width 0.25) (layer "B.Cu") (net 14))
 (segment (start 144.1 108.2) (end 143 108.2) (width 0.25) (layer "B.Cu") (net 14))
 (segment (start 131.872792 108.2) (end 131.236396 108.836396) (width 0.25) (layer "B.Cu") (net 14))
 (segment (start 131.236396 108.836396) (end 130.072789 110.000003) (width 0.25) (layer "B.Cu") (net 14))
 (segment (start 147.9 112) (end 144.1 108.2) (width 0.25) (layer "B.Cu") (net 14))
 (segment (start 130.072789 110.000003) (end 126 110.000003) (width 0.25) (layer "B.Cu") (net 14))
 (segment (start 158.943198 117.2) (end 156.393198 117.2) (width 0.25) (layer "F.Cu") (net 17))
 (segment (start 158.943198 117.2) (end 160.993198 117.2) (width 0.25) (layer "F.Cu") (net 17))
 (segment (start 132.27787 110.870839) (end 132.248709 110.9) (width 0.25) (layer "F.Cu") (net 17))
 (segment (start 132.248709 110.9) (end 128.1 110.9) (width 0.25) (layer "F.Cu") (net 17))
 (via (at 158.943198 117.2) (size 0.8) (drill 0.4) (layers "F.Cu" "B.Cu") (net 17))
 (via (at 132.27787 110.870839) (size 0.8) (drill 0.4) (layers "F.Cu" "B.Cu") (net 17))
 (segment (start 147.875153 116.524847) (end 146.081802 114.731496) (width 0.25) (layer "B.Cu") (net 17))
 (segment (start 160.418198 116.225) (end 160.418198 115.6) (width 0.2) (layer "B.Cu") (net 17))
 (segment (start 143.540812 109.55) (end 141.713604 109.55) (width 0.25) (layer "B.Cu") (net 17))
 (segment (start 150.8 118.375) (end 149.725306 118.375) (width 0.25) (layer "B.Cu") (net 17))
 (segment (start 149.725306 118.375) (end 147.875153 116.524847) (width 0.25) (layer "B.Cu") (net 17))
 (segment (start 158.943198 117.2) (end 157.768198 118.375) (width 0.25) (layer "B.Cu") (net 17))
 (segment (start 158.943198 116.575) (end 158.943198 117.2) (width 0.25) (layer "B.Cu") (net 17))
 (segment (start 145.445406 111.454594) (end 143.540812 109.55) (width 0.25) (layer "B.Cu") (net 17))
 (segment (start 141.713604 109.55) (end 133.598709 109.55) (width 0.25) (layer "B.Cu") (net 17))
 (segment (start 160.418198 115.1) (end 158.943198 116.575) (width 0.25) (layer "B.Cu") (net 17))
 (segment (start 146.081802 114.731496) (end 146.081802 113.3) (width 0.25) (layer "B.Cu") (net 17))
 (segment (start 146.081802 112.09099) (end 145.445406 111.454594) (width 0.25) (layer "B.Cu") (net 17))
 (segment (start 146.081802 113.3) (end 146.081802 112.09099) (width 0.25) (layer "B.Cu") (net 17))
 (segment (start 133.598709 109.55) (end 132.27787 110.870839) (width 0.25) (layer "B.Cu") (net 17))
 (segment (start 157.768198 118.375) (end 150.8 118.375) (width 0.25) (layer "B.Cu") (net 17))
 (segment (start 124.800006 111.000006) (end 124.7 110.9) (width 0.25) (layer "F.Cu") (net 16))
 (segment (start 156.393198 113) (end 155.393198 114) (width 0.25) (layer "F.Cu") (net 16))
 (segment (start 126 111.000006) (end 124.800006 111.000006) (width 0.25) (layer "F.Cu") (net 16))
 (segment (start 156.393198 113) (end 160.993198 113) (width 0.25) (layer "F.Cu") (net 16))
 (via (at 126 111.000006) (size 0.8) (drill 0.4) (layers "F.Cu" "B.Cu") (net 16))
 (via (at 155.393198 114) (size 0.8) (drill 0.4) (layers "F.Cu" "B.Cu") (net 16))
 (segment (start 146.531802 114.5451) (end 146.531802 111.904594) (width 0.25) (layer "B.Cu") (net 16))
 (segment (start 146.531802 111.904594) (end 143.727208 109.1) (width 0.25) (layer "B.Cu") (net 16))
 (segment (start 149.911702 117.925) (end 146.531802 114.5451) (width 0.25) (layer "B.Cu") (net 16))
 (segment (start 133.023403 109.1) (end 131.123397 111.000006) (width 0.25) (layer "B.Cu") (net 16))
 (segment (start 131.123397 111.000006) (end 126 111.000006) (width 0.25) (layer "B.Cu") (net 16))
 (segment (start 155.393198 114) (end 155.393198 114.8701) (width 0.25) (layer "B.Cu") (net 16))
 (segment (start 143.727208 109.1) (end 133.023403 109.1) (width 0.25) (layer "B.Cu") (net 16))
 (segment (start 152.338298 117.925) (end 149.911702 117.925) (width 0.25) (layer "B.Cu") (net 16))
 (segment (start 155.393198 114.8701) (end 152.338298 117.925) (width 0.25) (layer "B.Cu") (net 16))
 (segment (start 133.712653 111.712653) (end 133.7 111.7) (width 0.25) (layer "F.Cu") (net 19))
 (segment (start 166.443198 117.2) (end 168.493198 117.2) (width 0.25) (layer "F.Cu") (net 19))
 (segment (start 166.443198 117.2) (end 163.893198 117.2) (width 0.25) (layer "F.Cu") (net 19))
 (segment (start 133.7 111.7) (end 128.1 111.7) (width 0.25) (layer "F.Cu") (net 19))
 (via (at 133.712653 111.712653) (size 0.8) (drill 0.4) (layers "F.Cu" "B.Cu") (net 19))
 (via (at 166.443198 117.2) (size 0.8) (drill 0.4) (layers "F.Cu" "B.Cu") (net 19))
 (segment (start 167.918198 115.1) (end 166.443198 116.575) (width 0.25) (layer "B.Cu") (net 19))
 (segment (start 145.181802 112.463782) (end 144.70901 111.99099) (width 0.25) (layer "B.Cu") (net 19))
 (segment (start 148.438757 118.361243) (end 145.181802 115.104288) (width 0.25) (layer "B.Cu") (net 19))
 (segment (start 134.975306 110.45) (end 133.712653 111.712653) (width 0.25) (layer "B.Cu") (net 19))
 (segment (start 144.70901 111.99099) (end 143.16802 110.45) (width 0.25) (layer "B.Cu") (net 19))
 (segment (start 166.2 117.2) (end 164.125 119.275) (width 0.25) (layer "B.Cu") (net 19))
 (segment (start 159.151902 119.275) (end 149.352514 119.275) (width 0.25) (layer "B.Cu") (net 19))
 (segment (start 166.443198 116.575) (end 166.443198 117.2) (width 0.25) (layer "B.Cu") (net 19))
 (segment (start 145.181802 115.104288) (end 145.181802 113.9) (width 0.25) (layer "B.Cu") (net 19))
 (segment (start 166.443198 117.2) (end 166.2 117.2) (width 0.25) (layer "B.Cu") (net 19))
 (segment (start 164.125 119.275) (end 159.151902 119.275) (width 0.25) (layer "B.Cu") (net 19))
 (segment (start 149.352514 119.275) (end 148.438757 118.361243) (width 0.25) (layer "B.Cu") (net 19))
 (segment (start 145.181802 113.9) (end 145.181802 112.463782) (width 0.25) (layer "B.Cu") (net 19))
 (segment (start 141 110.45) (end 134.975306 110.45) (width 0.25) (layer "B.Cu") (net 19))
 (segment (start 143.16802 110.45) (end 141 110.45) (width 0.25) (layer "B.Cu") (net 19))
 (segment (start 125.699991 111.7) (end 124.7 111.7) (width 0.25) (layer "F.Cu") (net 18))
 (segment (start 163.893198 113) (end 168.493198 113) (width 0.25) (layer "F.Cu") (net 18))
 (segment (start 163.893198 113) (end 162.893198 114) (width 0.25) (layer "F.Cu") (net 18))
 (segment (start 126 112.000009) (end 125.699991 111.7) (width 0.25) (layer "F.Cu") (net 18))
 (via (at 162.893198 114) (size 0.8) (drill 0.4) (layers "F.Cu" "B.Cu") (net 18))
 (via (at 126 112.000009) (size 0.8) (drill 0.4) (layers "F.Cu" "B.Cu") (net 18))
 (segment (start 134.4 110) (end 132.399991 112.000009) (width 0.25) (layer "B.Cu") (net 18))
 (segment (start 145.631802 114.5451) (end 145.631802 112.277386) (width 0.25) (layer "B.Cu") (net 18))
 (segment (start 149.53891 118.825) (end 149.275306 118.561396) (width 0.25) (layer "B.Cu") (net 18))
 (segment (start 145.631802 114.917892) (end 145.631802 114.5451) (width 0.25) (layer "B.Cu") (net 18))
 (segment (start 149.275306 118.561396) (end 145.631802 114.917892) (width 0.25) (layer "B.Cu") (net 18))
 (segment (start 159.338298 118.825) (end 156.8 118.825) (width 0.25) (layer "B.Cu") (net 18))
 (segment (start 132.399991 112.000009) (end 126 112.000009) (width 0.25) (layer "B.Cu") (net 18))
 (segment (start 143.354416 110) (end 140.8 110) (width 0.25) (layer "B.Cu") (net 18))
 (segment (start 162.893198 115.2701) (end 159.338298 118.825) (width 0.25) (layer "B.Cu") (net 18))
 (segment (start 156.8 118.825) (end 149.53891 118.825) (width 0.25) (layer "B.Cu") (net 18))
 (segment (start 135.3 110) (end 134.4 110) (width 0.25) (layer "B.Cu") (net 18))
 (segment (start 144.677208 111.322792) (end 143.354416 110) (width 0.25) (layer "B.Cu") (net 18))
 (segment (start 145.631802 112.277386) (end 144.677208 111.322792) (width 0.25) (layer "B.Cu") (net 18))
 (segment (start 162.893198 114) (end 162.893198 115.2701) (width 0.25) (layer "B.Cu") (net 18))
 (segment (start 140.8 110) (end 135.3 110) (width 0.25) (layer "B.Cu") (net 18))
 (segment (start 126.4 113.4) (end 127.2 113.4) (width 0.25) (layer "F.Cu") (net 3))
 (segment (start 145 105) (end 143.65 105) (width 0.2) (layer "F.Cu") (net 3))
 (segment (start 142.35 106.3) (end 142.35 108.5) (width 0.2) (layer "F.Cu") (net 3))
 (segment (start 115 104) (end 112.5 106.5) (width 0.25) (layer "F.Cu") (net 3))
 (segment (start 134.9 105.675) (end 134.9 111.550611) (width 0.25) (layer "F.Cu") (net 3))
 (segment (start 113.9 113.4) (end 125.6 113.4) (width 0.25) (layer "F.Cu") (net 3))
 (segment (start 134.9 111.550611) (end 133.050611 113.4) (width 0.25) (layer "F.Cu") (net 3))
 (segment (start 133.050611 113.4) (end 127.2 113.4) (width 0.25) (layer "F.Cu") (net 3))
 (segment (start 143 108.5) (end 142.35 108.5) (width 0.2) (layer "F.Cu") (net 3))
 (segment (start 112.5 112) (end 113.9 113.4) (width 0.25) (layer "F.Cu") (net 3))
 (segment (start 112.5 106.5) (end 112.5 112) (width 0.25) (layer "F.Cu") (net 3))
 (segment (start 124.7 112.5) (end 125.6 113.4) (width 0.25) (layer "F.Cu") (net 3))
 (segment (start 125.6 113.4) (end 126.4 113.4) (width 0.25) (layer "F.Cu") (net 3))
 (segment (start 143.65 105) (end 142.35 106.3) (width 0.2) (layer "F.Cu") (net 3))
 (segment (start 144.9 105.1) (end 145 105) (width 0.2) (layer "F.Cu") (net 3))
 (segment (start 127.2 113.4) (end 128.1 112.5) (width 0.25) (layer "F.Cu") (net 3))
 (via (at 145 105) (size 0.6) (drill 0.3) (layers "F.Cu" "B.Cu") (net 3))
 (via (at 134.9 105.675) (size 0.8) (drill 0.4) (layers "F.Cu" "B.Cu") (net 3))
 (segment (start 145 105.95) (end 135.175 105.95) (width 0.25) (layer "B.Cu") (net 3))
 (segment (start 145 105) (end 145 105.95) (width 0.2) (layer "B.Cu") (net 3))
 (segment (start 135.175 105.95) (end 134.9 105.675) (width 0.25) (layer "B.Cu") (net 3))
 (segment (start 145.601 104.751057) (end 142.748943 101.899) (width 0.2) (layer "F.Cu") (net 2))
 (segment (start 122.181 101.899) (end 115 109.08) (width 0.2) (layer "F.Cu") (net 2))
 (segment (start 145.601 105.248943) (end 145.601 104.751057) (width 0.2) (layer "F.Cu") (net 2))
 (segment (start 142.748943 101.899) (end 122.181 101.899) (width 0.2) (layer "F.Cu") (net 2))
 (segment (start 143.65 106.3) (end 144.549943 106.3) (width 0.2) (layer "F.Cu") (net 2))
 (segment (start 144.549943 106.3) (end 145.601 105.248943) (width 0.2) (layer "F.Cu") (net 2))
 (segment (start 116.96 106.54) (end 115 106.54) (width 0.2) (layer "F.Cu") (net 1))
 (segment (start 143.65 108.5) (end 146.002 106.148) (width 0.2) (layer "F.Cu") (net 1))
 (segment (start 142.915043 101.498) (end 122.002 101.498) (width 0.2) (layer "F.Cu") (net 1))
 (segment (start 146.002 104.584957) (end 142.915043 101.498) (width 0.2) (layer "F.Cu") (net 1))
 (segment (start 122.002 101.498) (end 116.96 106.54) (width 0.2) (layer "F.Cu") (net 1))
 (segment (start 146.002 106.148) (end 146.002 104.584957) (width 0.2) (layer "F.Cu") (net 1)))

